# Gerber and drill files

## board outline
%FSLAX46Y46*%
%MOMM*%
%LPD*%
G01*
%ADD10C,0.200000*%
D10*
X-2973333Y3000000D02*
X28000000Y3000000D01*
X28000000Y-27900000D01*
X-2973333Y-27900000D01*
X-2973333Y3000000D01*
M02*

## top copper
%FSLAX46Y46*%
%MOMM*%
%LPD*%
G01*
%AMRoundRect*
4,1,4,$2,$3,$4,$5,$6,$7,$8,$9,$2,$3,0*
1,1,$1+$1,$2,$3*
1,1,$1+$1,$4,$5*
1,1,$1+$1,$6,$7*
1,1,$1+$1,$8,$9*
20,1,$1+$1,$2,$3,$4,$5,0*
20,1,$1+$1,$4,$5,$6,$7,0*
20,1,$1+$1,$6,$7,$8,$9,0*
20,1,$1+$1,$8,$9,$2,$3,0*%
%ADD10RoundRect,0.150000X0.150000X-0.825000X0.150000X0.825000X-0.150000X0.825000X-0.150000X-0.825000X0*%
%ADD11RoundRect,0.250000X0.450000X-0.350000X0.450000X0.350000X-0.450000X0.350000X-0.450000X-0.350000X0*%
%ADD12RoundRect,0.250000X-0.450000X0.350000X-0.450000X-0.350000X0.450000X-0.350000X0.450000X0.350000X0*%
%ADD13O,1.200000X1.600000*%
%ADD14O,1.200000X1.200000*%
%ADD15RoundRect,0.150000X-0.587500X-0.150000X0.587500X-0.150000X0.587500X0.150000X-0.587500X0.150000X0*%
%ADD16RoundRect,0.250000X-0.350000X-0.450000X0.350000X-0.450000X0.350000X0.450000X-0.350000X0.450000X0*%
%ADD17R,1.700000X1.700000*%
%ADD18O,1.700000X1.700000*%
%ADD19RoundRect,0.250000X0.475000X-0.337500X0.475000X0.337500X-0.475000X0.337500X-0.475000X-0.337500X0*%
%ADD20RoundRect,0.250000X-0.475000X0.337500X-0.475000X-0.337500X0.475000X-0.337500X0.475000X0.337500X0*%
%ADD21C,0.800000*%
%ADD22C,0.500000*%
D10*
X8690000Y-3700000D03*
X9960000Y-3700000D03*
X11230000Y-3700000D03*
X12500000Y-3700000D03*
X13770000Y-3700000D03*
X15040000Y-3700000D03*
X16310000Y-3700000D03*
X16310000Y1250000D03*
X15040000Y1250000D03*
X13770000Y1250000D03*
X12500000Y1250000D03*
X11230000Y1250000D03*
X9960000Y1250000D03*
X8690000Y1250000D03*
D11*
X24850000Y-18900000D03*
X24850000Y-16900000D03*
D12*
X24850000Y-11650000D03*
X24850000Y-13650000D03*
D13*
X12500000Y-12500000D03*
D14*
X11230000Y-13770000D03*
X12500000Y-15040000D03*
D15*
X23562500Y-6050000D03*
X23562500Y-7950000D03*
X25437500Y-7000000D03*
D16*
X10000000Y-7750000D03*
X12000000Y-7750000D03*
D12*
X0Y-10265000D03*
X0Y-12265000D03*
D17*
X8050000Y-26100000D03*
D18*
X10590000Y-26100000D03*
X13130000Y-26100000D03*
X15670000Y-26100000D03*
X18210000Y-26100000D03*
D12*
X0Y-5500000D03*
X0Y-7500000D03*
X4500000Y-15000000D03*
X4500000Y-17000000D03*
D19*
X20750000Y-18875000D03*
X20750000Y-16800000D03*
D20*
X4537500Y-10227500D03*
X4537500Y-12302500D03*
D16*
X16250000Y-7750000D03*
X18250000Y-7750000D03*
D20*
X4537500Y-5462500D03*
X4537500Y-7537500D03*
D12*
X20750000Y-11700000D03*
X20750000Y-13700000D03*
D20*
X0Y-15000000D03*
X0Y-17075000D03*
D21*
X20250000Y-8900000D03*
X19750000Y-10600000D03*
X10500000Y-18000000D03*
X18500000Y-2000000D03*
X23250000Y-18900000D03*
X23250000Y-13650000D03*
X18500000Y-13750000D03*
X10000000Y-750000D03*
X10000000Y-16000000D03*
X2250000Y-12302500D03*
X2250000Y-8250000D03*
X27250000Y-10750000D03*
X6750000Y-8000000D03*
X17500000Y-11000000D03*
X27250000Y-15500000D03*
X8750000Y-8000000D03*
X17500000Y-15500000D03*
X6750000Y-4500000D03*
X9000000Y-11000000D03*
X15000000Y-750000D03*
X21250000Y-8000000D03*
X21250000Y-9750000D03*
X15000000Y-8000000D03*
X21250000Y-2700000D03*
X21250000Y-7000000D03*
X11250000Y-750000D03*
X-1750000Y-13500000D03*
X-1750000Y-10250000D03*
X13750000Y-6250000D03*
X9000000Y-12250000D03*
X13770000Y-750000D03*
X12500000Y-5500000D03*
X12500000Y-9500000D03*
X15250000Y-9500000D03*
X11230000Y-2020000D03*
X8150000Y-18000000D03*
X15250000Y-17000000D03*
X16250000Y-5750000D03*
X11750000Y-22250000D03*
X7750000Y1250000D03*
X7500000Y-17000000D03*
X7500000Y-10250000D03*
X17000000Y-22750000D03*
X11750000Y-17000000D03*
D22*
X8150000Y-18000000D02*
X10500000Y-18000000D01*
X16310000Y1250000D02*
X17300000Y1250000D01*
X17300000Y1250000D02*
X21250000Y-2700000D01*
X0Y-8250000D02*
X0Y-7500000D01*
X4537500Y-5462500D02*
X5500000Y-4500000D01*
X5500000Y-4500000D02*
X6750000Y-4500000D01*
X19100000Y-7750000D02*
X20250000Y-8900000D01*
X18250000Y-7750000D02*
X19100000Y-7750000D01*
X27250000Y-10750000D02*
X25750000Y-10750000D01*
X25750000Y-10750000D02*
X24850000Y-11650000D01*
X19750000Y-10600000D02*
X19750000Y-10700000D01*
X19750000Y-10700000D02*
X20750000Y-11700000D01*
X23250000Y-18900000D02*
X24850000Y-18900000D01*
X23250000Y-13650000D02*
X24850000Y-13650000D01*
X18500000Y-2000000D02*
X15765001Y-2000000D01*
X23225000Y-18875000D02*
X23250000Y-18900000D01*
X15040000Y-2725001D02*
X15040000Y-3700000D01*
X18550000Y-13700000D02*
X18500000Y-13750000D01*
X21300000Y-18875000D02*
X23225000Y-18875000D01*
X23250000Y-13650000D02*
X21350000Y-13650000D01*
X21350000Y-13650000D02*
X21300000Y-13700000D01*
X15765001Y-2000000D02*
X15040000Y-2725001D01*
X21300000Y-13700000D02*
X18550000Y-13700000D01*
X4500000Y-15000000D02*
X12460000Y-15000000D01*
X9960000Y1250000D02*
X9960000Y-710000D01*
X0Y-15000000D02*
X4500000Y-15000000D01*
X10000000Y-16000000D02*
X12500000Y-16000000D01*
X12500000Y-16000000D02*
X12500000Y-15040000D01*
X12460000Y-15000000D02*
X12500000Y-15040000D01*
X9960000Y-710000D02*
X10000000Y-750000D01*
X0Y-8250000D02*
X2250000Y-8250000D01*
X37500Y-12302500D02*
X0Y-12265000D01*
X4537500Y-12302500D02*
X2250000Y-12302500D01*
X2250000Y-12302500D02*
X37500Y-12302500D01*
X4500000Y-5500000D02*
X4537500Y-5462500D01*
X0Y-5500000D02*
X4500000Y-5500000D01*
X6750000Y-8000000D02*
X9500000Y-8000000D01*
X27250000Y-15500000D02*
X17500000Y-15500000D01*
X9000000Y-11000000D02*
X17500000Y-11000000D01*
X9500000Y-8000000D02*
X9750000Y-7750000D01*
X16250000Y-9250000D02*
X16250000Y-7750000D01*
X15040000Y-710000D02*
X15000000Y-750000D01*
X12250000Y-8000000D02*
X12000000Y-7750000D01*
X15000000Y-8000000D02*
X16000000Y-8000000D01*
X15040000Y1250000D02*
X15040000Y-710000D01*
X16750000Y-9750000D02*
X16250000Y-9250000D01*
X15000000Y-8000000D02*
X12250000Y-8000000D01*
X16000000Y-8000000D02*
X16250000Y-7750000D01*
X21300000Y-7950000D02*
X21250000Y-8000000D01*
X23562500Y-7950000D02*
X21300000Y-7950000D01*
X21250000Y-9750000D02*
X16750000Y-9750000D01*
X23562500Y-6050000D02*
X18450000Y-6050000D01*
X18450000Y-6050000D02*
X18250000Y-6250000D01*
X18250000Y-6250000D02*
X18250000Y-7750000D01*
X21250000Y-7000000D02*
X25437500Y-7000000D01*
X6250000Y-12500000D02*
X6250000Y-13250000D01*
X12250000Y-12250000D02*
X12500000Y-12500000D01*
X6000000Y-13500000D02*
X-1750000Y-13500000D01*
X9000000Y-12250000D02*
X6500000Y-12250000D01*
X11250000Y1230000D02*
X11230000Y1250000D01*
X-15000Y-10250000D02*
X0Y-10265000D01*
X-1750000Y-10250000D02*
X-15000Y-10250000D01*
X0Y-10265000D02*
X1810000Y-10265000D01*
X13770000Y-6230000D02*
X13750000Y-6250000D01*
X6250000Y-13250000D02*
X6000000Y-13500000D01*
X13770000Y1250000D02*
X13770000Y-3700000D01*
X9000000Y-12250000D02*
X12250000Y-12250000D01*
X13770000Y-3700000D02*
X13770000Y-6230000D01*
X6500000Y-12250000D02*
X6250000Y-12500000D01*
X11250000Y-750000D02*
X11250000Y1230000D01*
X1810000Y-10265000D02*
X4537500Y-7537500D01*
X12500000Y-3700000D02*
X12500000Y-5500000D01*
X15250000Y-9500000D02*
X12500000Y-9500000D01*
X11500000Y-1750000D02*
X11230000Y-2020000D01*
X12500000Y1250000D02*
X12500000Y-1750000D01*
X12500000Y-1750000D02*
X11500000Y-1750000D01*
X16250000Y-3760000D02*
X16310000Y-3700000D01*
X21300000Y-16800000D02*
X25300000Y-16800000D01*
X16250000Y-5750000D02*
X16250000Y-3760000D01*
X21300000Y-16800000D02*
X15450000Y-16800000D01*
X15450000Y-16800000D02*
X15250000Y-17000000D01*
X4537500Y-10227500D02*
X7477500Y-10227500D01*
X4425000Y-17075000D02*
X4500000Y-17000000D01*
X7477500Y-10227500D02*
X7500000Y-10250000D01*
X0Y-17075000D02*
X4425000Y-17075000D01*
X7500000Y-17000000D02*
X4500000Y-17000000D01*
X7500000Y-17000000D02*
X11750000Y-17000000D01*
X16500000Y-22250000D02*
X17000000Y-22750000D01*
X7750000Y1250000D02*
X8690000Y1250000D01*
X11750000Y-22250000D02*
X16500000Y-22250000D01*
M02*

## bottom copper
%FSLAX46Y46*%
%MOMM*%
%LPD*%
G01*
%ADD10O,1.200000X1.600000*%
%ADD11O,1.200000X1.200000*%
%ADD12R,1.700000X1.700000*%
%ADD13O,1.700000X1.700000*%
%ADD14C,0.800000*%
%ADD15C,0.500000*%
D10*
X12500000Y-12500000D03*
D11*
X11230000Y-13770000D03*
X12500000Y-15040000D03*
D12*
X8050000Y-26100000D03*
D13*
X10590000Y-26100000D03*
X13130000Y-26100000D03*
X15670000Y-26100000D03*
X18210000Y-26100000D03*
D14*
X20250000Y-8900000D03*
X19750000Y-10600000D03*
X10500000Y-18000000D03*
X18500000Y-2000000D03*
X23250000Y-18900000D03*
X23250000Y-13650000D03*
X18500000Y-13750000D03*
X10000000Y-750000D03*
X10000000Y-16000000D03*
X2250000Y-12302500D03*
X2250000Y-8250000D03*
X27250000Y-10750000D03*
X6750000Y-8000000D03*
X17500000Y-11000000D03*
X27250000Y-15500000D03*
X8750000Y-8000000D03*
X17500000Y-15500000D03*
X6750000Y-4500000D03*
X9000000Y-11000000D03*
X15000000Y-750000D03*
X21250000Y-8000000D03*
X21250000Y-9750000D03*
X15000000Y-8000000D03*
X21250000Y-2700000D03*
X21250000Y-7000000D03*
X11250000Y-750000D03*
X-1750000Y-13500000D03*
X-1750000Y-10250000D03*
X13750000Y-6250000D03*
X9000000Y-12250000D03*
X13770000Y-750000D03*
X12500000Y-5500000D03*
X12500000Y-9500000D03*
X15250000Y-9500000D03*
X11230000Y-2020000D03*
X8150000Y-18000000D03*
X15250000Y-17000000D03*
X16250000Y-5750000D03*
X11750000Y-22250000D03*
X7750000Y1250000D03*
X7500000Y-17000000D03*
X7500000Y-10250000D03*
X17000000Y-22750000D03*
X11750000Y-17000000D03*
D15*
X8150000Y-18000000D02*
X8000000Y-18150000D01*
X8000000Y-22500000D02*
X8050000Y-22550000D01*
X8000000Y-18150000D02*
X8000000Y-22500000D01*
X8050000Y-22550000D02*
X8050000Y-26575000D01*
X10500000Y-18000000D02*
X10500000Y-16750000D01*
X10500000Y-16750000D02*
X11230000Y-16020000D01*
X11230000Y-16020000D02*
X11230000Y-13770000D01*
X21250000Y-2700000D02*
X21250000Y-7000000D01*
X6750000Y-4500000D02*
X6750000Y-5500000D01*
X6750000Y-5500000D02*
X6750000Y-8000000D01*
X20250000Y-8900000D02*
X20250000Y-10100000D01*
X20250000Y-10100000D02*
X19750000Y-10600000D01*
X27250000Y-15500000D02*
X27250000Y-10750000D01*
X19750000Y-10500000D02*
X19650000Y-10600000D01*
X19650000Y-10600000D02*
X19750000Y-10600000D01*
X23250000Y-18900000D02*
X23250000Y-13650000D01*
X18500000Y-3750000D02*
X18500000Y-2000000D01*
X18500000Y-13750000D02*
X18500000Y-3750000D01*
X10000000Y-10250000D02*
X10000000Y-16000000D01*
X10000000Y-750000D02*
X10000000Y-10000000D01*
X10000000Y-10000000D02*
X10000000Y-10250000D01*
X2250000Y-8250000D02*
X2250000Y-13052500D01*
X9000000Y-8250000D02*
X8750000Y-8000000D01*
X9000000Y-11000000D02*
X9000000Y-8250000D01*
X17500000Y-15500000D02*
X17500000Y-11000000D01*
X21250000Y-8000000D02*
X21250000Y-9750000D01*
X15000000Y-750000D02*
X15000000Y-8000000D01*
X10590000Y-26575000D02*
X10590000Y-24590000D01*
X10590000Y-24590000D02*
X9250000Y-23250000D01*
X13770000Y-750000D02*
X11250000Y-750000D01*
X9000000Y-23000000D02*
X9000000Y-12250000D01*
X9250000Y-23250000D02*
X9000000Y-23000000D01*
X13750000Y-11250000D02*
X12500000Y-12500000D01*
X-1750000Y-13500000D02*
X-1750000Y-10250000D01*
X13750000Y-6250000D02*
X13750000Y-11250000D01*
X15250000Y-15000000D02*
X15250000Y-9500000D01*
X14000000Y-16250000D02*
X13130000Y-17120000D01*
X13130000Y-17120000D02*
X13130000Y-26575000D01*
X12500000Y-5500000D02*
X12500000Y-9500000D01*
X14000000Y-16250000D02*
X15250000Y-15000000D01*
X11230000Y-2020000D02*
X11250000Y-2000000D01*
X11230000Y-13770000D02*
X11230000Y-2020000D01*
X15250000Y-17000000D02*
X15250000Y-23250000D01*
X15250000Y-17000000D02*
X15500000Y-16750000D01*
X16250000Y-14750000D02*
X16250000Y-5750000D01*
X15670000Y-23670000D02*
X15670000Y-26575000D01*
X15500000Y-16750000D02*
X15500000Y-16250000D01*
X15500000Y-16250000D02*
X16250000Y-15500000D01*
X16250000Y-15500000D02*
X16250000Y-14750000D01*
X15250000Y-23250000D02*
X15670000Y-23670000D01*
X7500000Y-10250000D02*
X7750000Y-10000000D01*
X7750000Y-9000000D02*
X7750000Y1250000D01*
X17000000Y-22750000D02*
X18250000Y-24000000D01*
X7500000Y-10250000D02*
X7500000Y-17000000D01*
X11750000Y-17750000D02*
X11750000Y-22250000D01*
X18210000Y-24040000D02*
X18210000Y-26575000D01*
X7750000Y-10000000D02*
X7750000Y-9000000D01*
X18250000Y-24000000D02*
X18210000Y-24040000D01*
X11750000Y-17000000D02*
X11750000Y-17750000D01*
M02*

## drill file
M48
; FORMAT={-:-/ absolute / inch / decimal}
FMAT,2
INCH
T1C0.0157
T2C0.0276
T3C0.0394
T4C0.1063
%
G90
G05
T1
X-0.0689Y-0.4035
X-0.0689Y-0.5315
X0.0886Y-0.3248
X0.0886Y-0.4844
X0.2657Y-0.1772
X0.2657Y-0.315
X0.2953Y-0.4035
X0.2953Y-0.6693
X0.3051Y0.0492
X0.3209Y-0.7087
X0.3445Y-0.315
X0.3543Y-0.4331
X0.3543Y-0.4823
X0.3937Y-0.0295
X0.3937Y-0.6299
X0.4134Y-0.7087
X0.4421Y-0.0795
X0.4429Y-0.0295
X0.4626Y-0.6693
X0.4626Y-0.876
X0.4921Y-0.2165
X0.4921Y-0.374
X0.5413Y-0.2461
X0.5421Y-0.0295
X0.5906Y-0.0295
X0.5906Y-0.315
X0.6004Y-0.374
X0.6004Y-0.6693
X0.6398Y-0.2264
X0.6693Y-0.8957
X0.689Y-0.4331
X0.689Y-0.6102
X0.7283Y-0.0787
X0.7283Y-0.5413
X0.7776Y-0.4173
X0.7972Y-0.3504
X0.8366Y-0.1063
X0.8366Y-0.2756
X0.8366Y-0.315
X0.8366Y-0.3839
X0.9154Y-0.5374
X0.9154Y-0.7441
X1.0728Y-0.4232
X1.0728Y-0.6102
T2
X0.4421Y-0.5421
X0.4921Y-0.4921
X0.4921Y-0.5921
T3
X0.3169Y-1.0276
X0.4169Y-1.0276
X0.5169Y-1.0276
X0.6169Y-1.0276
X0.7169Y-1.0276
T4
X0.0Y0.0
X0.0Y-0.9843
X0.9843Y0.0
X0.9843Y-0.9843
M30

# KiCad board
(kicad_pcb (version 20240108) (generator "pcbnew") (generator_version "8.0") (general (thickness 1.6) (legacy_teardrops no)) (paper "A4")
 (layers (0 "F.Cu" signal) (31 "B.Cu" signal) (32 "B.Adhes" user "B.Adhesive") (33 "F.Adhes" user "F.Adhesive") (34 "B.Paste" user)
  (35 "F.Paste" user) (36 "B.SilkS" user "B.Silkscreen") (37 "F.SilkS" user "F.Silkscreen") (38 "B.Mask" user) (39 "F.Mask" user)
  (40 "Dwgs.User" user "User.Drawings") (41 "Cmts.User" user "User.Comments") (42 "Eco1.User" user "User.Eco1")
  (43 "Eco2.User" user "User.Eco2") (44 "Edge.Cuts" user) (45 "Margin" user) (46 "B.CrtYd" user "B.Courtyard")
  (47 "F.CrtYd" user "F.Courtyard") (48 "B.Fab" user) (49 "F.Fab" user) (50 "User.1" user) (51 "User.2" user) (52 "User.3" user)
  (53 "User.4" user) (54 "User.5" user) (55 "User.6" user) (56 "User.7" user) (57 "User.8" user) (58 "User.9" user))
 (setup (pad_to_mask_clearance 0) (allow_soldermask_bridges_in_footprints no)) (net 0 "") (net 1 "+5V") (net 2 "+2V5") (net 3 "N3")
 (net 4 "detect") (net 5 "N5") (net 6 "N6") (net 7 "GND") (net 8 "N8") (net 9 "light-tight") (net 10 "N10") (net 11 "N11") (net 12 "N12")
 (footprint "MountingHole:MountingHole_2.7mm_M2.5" (layer "F.Cu") (at 0 0)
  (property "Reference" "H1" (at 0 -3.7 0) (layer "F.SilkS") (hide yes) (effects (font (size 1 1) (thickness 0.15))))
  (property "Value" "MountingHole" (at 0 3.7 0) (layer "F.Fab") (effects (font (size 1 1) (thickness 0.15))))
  (pad "" np_thru_hole circle (at 0 0) (size 2.7 2.7) (drill 2.7) (layers "*.Cu" "*.Mask")))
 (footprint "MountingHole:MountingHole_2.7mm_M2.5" (layer "F.Cu") (at 0 25)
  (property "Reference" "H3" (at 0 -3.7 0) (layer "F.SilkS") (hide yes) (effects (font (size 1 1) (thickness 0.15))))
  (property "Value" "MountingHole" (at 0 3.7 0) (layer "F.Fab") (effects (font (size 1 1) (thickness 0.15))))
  (pad "" np_thru_hole circle (at 0 0) (size 2.7 2.7) (drill 2.7) (layers "*.Cu" "*.Mask")))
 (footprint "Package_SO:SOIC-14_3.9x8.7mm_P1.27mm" (layer "F.Cu") (at 12.5 1.225 90)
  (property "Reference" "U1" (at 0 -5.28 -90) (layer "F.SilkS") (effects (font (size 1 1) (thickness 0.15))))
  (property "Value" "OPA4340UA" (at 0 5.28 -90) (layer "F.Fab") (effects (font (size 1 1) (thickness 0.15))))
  (pad "1" smd roundrect (at -2.475 -3.81 90) (size 1.95 0.6) (layers "F.Cu" "F.Paste" "F.Mask") (roundrect_rratio 0.25))
  (pad "2" smd roundrect (at -2.475 -2.54 90) (size 1.95 0.6) (layers "F.Cu" "F.Paste" "F.Mask") (roundrect_rratio 0.25))
  (pad "3" smd roundrect (at -2.475 -1.27 90) (size 1.95 0.6) (layers "F.Cu" "F.Paste" "F.Mask") (roundrect_rratio 0.25))
  (pad "4" smd roundrect (at -2.475 0 90) (size 1.95 0.6) (layers "F.Cu" "F.Paste" "F.Mask") (roundrect_rratio 0.25) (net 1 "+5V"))
  (pad "5" smd roundrect (at -2.475 1.27 90) (size 1.95 0.6) (layers "F.Cu" "F.Paste" "F.Mask") (roundrect_rratio 0.25) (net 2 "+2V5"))
  (pad "6" smd roundrect (at -2.475 2.54 90) (size 1.95 0.6) (layers "F.Cu" "F.Paste" "F.Mask") (roundrect_rratio 0.25) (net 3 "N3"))
  (pad "7" smd roundrect (at -2.475 3.81 90) (size 1.95 0.6) (layers "F.Cu" "F.Paste" "F.Mask") (roundrect_rratio 0.25) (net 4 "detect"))
  (pad "8" smd roundrect (at 2.475 3.81 90) (size 1.95 0.6) (layers "F.Cu" "F.Paste" "F.Mask") (roundrect_rratio 0.25) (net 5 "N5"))
  (pad "9" smd roundrect (at 2.475 2.54 90) (size 1.95 0.6) (layers "F.Cu" "F.Paste" "F.Mask") (roundrect_rratio 0.25) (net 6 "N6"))
  (pad "10" smd roundrect (at 2.475 1.27 90) (size 1.95 0.6) (layers "F.Cu" "F.Paste" "F.Mask") (roundrect_rratio 0.25) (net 2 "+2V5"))
  (pad "11" smd roundrect (at 2.475 0 90) (size 1.95 0.6) (layers "F.Cu" "F.Paste" "F.Mask") (roundrect_rratio 0.25) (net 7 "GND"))
  (pad "12" smd roundrect (at 2.475 -1.27 90) (size 1.95 0.6) (layers "F.Cu" "F.Paste" "F.Mask") (roundrect_rratio 0.25) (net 2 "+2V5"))
  (pad "13" smd roundrect (at 2.475 -2.54 90) (size 1.95 0.6) (layers "F.Cu" "F.Paste" "F.Mask") (roundrect_rratio 0.25) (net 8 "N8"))
  (pad "14" smd roundrect (at 2.475 -3.81 90) (size 1.95 0.6) (layers "F.Cu" "F.Paste" "F.Mask") (roundrect_rratio 0.25)
   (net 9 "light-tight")))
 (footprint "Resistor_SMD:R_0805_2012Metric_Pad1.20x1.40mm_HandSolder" (layer "F.Cu") (at 24.85 17.9 90)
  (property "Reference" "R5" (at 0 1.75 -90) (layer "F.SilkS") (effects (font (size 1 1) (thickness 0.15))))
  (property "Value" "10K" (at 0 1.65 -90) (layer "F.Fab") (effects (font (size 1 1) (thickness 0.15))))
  (pad "1" smd roundrect (at -1 0 90) (size 1.2 1.4) (layers "F.Cu" "F.Paste" "F.Mask") (roundrect_rratio 0.208333) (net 3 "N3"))
  (pad "2" smd roundrect (at 1 0 90) (size 1.2 1.4) (layers "F.Cu" "F.Paste" "F.Mask") (roundrect_rratio 0.208333) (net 4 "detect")))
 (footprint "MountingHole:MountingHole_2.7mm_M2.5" (layer "F.Cu") (at 25 25)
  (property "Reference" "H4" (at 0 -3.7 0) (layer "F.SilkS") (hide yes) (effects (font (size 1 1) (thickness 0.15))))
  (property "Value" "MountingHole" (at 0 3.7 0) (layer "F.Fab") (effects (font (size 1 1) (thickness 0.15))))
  (pad "" np_thru_hole circle (at 0 0) (size 2.7 2.7) (drill 2.7) (layers "*.Cu" "*.Mask")))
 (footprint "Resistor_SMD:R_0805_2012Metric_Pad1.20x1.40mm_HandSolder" (layer "F.Cu") (at 24.85 12.65 -90)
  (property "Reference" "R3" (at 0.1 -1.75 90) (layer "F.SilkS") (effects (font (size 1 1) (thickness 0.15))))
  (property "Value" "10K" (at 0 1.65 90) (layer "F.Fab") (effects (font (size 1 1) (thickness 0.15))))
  (pad "1" smd roundrect (at -1 0 270) (size 1.2 1.4) (layers "F.Cu" "F.Paste" "F.Mask") (roundrect_rratio 0.208333) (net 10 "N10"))
  (pad "2" smd roundrect (at 1 0 270) (size 1.2 1.4) (layers "F.Cu" "F.Paste" "F.Mask") (roundrect_rratio 0.208333) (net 3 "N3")))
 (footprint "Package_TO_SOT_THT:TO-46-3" (layer "F.Cu") (at 12.5 12.5 -90)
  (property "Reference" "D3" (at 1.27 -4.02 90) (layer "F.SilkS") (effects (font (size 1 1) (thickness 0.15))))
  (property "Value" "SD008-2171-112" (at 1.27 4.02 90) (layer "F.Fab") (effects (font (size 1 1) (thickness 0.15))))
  (pad "1" thru_hole oval (at 0 0 270) (size 1.6 1.2) (drill 0.7) (layers "*.Cu" "*.Mask") (remove_unused_layers no) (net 2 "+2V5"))
  (pad "2" thru_hole oval (at 1.27 1.27 270) (size 1.2 1.2) (drill 0.7) (layers "*.Cu" "*.Mask") (remove_unused_layers no) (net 7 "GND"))
  (pad "3" thru_hole oval (at 2.54 0 270) (size 1.2 1.2) (drill 0.7) (layers "*.Cu" "*.Mask") (remove_unused_layers no) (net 8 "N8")))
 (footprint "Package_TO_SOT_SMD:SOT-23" (layer "F.Cu") (at 24.5 7)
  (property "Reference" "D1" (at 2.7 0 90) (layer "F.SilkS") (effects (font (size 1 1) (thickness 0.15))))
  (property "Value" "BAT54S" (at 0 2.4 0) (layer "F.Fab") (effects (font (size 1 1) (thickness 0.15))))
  (pad "1" smd roundrect (at -0.9375 -0.95) (size 1.475 0.6) (layers "F.Cu" "F.Paste" "F.Mask") (roundrect_rratio 0.25) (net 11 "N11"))
  (pad "2" smd roundrect (at -0.9375 0.95) (size 1.475 0.6) (layers "F.Cu" "F.Paste" "F.Mask") (roundrect_rratio 0.25) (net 6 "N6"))
  (pad "3" smd roundrect (at 0.9375 0) (size 1.475 0.6) (layers "F.Cu" "F.Paste" "F.Mask") (roundrect_rratio 0.25) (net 5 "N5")))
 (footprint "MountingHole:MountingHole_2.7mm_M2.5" (layer "F.Cu") (at 25 0)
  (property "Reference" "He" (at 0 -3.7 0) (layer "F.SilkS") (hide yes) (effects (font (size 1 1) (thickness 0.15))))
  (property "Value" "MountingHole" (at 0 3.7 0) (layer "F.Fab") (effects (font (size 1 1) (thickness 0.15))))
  (pad "" np_thru_hole circle (at 0 0) (size 2.7 2.7) (drill 2.7) (layers "*.Cu" "*.Mask")))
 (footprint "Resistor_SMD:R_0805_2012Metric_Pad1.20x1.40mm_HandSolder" (layer "F.Cu") (at 11 7.75)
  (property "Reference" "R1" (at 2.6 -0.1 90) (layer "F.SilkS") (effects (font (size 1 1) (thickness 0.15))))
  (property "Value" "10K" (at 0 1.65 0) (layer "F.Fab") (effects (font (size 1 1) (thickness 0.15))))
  (pad "1" smd roundrect (at -1 0) (size 1.2 1.4) (layers "F.Cu" "F.Paste" "F.Mask") (roundrect_rratio 0.208333) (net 10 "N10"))
  (pad "2" smd roundrect (at 1 0) (size 1.2 1.4) (layers "F.Cu" "F.Paste" "F.Mask") (roundrect_rratio 0.208333) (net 6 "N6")))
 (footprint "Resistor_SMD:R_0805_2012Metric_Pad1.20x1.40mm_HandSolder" (layer "F.Cu") (at 0 11.265 -90)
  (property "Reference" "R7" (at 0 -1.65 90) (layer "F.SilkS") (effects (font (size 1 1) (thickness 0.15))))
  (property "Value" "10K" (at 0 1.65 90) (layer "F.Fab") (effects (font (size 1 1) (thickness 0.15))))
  (pad "1" smd roundrect (at -1 0 270) (size 1.2 1.4) (layers "F.Cu" "F.Paste" "F.Mask") (roundrect_rratio 0.208333) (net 2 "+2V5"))
  (pad "2" smd roundrect (at 1 0 270) (size 1.2 1.4) (layers "F.Cu" "F.Paste" "F.Mask") (roundrect_rratio 0.208333) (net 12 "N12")))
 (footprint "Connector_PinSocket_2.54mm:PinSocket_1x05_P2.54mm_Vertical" (layer "F.Cu") (at 8.05 26.1 90)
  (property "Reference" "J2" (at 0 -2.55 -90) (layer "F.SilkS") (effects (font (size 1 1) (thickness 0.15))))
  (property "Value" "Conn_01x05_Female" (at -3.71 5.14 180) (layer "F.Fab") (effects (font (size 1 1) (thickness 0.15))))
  (pad "1" thru_hole rect (at 0 0 90) (size 1.7 1.7) (drill 1) (layers "*.Cu" "*.Mask") (remove_unused_layers no) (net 7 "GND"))
  (pad "2" thru_hole oval (at 0 2.54 90) (size 1.7 1.7) (drill 1) (layers "*.Cu" "*.Mask") (remove_unused_layers no) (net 2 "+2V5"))
  (pad "3" thru_hole oval (at 0 5.08 90) (size 1.7 1.7) (drill 1) (layers "*.Cu" "*.Mask") (remove_unused_layers no) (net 1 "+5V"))
  (pad "4" thru_hole oval (at 0 7.62 90) (size 1.7 1.7) (drill 1) (layers "*.Cu" "*.Mask") (remove_unused_layers no) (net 4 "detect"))
  (pad "5" thru_hole oval (at 0 10.16 90) (size 1.7 1.7) (drill 1) (layers "*.Cu" "*.Mask") (remove_unused_layers no) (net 9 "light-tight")))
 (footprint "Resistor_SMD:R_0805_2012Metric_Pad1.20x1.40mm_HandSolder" (layer "F.Cu") (at 0 6.5 -90)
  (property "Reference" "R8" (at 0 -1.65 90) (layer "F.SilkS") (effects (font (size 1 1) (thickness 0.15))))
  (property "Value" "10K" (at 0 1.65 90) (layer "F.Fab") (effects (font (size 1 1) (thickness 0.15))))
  (pad "1" smd roundrect (at -1 0 270) (size 1.2 1.4) (layers "F.Cu" "F.Paste" "F.Mask") (roundrect_rratio 0.208333) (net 10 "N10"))
  (pad "2" smd roundrect (at 1 0 270) (size 1.2 1.4) (layers "F.Cu" "F.Paste" "F.Mask") (roundrect_rratio 0.208333) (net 12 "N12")))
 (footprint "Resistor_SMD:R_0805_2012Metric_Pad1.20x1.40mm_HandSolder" (layer "F.Cu") (at 4.5 16 -90)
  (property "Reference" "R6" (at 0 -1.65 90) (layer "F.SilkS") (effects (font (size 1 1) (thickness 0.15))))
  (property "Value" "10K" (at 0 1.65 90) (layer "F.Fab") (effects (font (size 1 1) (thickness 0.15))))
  (pad "1" smd roundrect (at -1 0 270) (size 1.2 1.4) (layers "F.Cu" "F.Paste" "F.Mask") (roundrect_rratio 0.208333) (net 8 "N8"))
  (pad "2" smd roundrect (at 1 0 270) (size 1.2 1.4) (layers "F.Cu" "F.Paste" "F.Mask") (roundrect_rratio 0.208333) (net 9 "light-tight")))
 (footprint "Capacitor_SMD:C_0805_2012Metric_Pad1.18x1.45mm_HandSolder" (layer "F.Cu") (at 20.75 17.8375 90)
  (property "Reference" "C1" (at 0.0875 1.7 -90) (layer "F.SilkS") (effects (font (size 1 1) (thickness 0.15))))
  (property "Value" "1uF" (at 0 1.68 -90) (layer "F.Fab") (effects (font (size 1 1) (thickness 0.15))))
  (pad "1" smd roundrect (at -1.0375 0 90) (size 1.175 1.45) (layers "F.Cu" "F.Paste" "F.Mask") (roundrect_rratio 0.212766) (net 3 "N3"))
  (pad "2" smd roundrect (at 1.0375 0 90) (size 1.175 1.45) (layers "F.Cu" "F.Paste" "F.Mask") (roundrect_rratio 0.212766) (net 4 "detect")))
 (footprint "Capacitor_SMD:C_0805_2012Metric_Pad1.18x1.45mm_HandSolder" (layer "F.Cu") (at 4.5375 11.265 -90)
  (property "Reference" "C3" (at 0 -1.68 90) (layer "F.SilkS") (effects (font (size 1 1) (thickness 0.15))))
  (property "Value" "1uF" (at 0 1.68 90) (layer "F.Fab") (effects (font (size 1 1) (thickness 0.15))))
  (pad "1" smd roundrect (at -1.0375 0 270) (size 1.175 1.45) (layers "F.Cu" "F.Paste" "F.Mask") (roundrect_rratio 0.212766)
   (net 9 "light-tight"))
  (pad "2" smd roundrect (at 1.0375 0 270) (size 1.175 1.45) (layers "F.Cu" "F.Paste" "F.Mask") (roundrect_rratio 0.212766) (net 12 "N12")))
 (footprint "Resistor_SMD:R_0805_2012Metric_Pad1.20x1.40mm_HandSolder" (layer "F.Cu") (at 17.25 7.75)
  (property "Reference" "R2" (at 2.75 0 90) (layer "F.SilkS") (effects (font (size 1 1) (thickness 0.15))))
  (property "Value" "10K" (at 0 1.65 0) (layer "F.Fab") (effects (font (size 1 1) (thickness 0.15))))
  (pad "1" smd roundrect (at -1 0) (size 1.2 1.4) (layers "F.Cu" "F.Paste" "F.Mask") (roundrect_rratio 0.208333) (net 6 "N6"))
  (pad "2" smd roundrect (at 1 0) (size 1.2 1.4) (layers "F.Cu" "F.Paste" "F.Mask") (roundrect_rratio 0.208333) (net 11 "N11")))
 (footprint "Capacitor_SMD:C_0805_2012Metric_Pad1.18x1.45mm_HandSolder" (layer "F.Cu") (at 4.5375 6.5 -90)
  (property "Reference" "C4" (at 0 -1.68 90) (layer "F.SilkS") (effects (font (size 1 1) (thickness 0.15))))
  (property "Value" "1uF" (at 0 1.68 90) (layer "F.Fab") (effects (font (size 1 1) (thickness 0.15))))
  (pad "1" smd roundrect (at -1.0375 0 270) (size 1.175 1.45) (layers "F.Cu" "F.Paste" "F.Mask") (roundrect_rratio 0.212766) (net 10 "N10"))
  (pad "2" smd roundrect (at 1.0375 0 270) (size 1.175 1.45) (layers "F.Cu" "F.Paste" "F.Mask") (roundrect_rratio 0.212766) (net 2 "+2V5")))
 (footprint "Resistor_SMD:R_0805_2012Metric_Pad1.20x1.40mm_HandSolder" (layer "F.Cu") (at 20.75 12.7 -90)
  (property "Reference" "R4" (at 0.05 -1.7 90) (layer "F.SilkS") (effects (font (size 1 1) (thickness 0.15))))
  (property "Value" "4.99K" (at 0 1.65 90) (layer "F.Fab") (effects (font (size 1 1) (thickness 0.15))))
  (pad "1" smd roundrect (at -1 0 270) (size 1.2 1.4) (layers "F.Cu" "F.Paste" "F.Mask") (roundrect_rratio 0.208333) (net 11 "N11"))
  (pad "2" smd roundrect (at 1 0 270) (size 1.2 1.4) (layers "F.Cu" "F.Paste" "F.Mask") (roundrect_rratio 0.208333) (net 3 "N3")))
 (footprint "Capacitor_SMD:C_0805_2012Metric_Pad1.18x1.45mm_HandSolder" (layer "F.Cu") (at 0 16.0375 -90)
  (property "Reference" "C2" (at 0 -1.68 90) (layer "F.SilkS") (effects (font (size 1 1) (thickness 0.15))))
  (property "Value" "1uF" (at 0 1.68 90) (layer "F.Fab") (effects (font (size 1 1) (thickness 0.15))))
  (pad "1" smd roundrect (at -1.0375 0 270) (size 1.175 1.45) (layers "F.Cu" "F.Paste" "F.Mask") (roundrect_rratio 0.212766) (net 8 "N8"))
  (pad "2" smd roundrect (at 1.0375 0 270) (size 1.175 1.45) (layers "F.Cu" "F.Paste" "F.Mask") (roundrect_rratio 0.212766)
   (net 9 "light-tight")))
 (gr_rect (start -2.973333 -3) (end 28 27.9) (stroke (width 0.2) (type default)) (fill none) (layer "Edge.Cuts"))
 (segment (start 23.25 18.9) (end 24.85 18.9) (width 0.5) (layer "F.Cu") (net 3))
 (segment (start 18.5 2) (end 15.765001 2) (width 0.5) (layer "F.Cu") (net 3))
 (segment (start 23.225 18.875) (end 23.25 18.9) (width 0.5) (layer "F.Cu") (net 3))
 (segment (start 15.04 2.725001) (end 15.04 3.7) (width 0.5) (layer "F.Cu") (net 3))
 (segment (start 18.55 13.7) (end 18.5 13.75) (width 0.5) (layer "F.Cu") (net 3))
 (segment (start 23.25 13.65) (end 24.85 13.65) (width 0.5) (layer "F.Cu") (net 3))
 (segment (start 21.3 18.875) (end 23.225 18.875) (width 0.5) (layer "F.Cu") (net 3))
 (segment (start 23.25 13.65) (end 21.35 13.65) (width 0.5) (layer "F.Cu") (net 3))
 (segment (start 21.35 13.65) (end 21.3 13.7) (width 0.5) (layer "F.Cu") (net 3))
 (segment (start 15.765001 2) (end 15.04 2.725001) (width 0.5) (layer "F.Cu") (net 3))
 (segment (start 21.3 13.7) (end 18.55 13.7) (width 0.5) (layer "F.Cu") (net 3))
 (via (at 18.5 2) (size 0.8) (drill 0.4) (layers "F.Cu" "B.Cu") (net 3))
 (via (at 23.25 18.9) (size 0.8) (drill 0.4) (layers "F.Cu" "B.Cu") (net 3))
 (via (at 23.25 13.65) (size 0.8) (drill 0.4) (layers "F.Cu" "B.Cu") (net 3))
 (via (at 18.5 13.75) (size 0.8) (drill 0.4) (layers "F.Cu" "B.Cu") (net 3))
 (segment (start 23.25 18.9) (end 23.25 13.65) (width 0.5) (layer "B.Cu") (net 3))
 (segment (start 18.5 3.75) (end 18.5 2) (width 0.5) (layer "B.Cu") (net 3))
 (segment (start 18.5 13.75) (end 18.5 3.75) (width 0.5) (layer "B.Cu") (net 3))
 (segment (start 4.5 15) (end 12.46 15) (width 0.5) (layer "F.Cu") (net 8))
 (segment (start 9.96 -1.25) (end 9.96 0.71) (width 0.5) (layer "F.Cu") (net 8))
 (segment (start 0 15) (end 4.5 15) (width 0.5) (layer "F.Cu") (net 8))
 (segment (start 10 16) (end 12.5 16) (width 0.5) (layer "F.Cu") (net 8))
 (segment (start 12.5 16) (end 12.5 15.04) (width 0.5) (layer "F.Cu") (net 8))
 (segment (start 12.46 15) (end 12.5 15.04) (width 0.5) (layer "F.Cu") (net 8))
 (segment (start 9.96 0.71) (end 10 0.75) (width 0.5) (layer "F.Cu") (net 8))
 (via (at 10 0.75) (size 0.8) (drill 0.4) (layers "F.Cu" "B.Cu") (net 8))
 (via (at 10 16) (size 0.8) (drill 0.4) (layers "F.Cu" "B.Cu") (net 8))
 (segment (start 10 10.25) (end 10 16) (width 0.5) (layer "B.Cu") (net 8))
 (segment (start 10 0.75) (end 10 10) (width 0.5) (layer "B.Cu") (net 8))
 (segment (start 10 10) (end 10 10.25) (width 0.5) (layer "B.Cu") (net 8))
 (segment (start 0 8.25) (end 2.25 8.25) (width 0.5) (layer "F.Cu") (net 12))
 (segment (start 0 8.25) (end 0 7.5) (width 0.5) (layer "F.Cu") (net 12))
 (segment (start 0.0375 12.3025) (end 0 12.265) (width 0.5) (layer "F.Cu") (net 12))
 (segment (start 4.5375 12.3025) (end 2.25 12.3025) (width 0.5) (layer "F.Cu") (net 12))
 (segment (start 2.25 12.3025) (end 0.0375 12.3025) (width 0.5) (layer "F.Cu") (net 12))
 (via (at 2.25 12.3025) (size 0.8) (drill 0.4) (layers "F.Cu" "B.Cu") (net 12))
 (via (at 2.25 8.25) (size 0.8) (drill 0.4) (layers "F.Cu" "B.Cu") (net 12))
 (segment (start 2.25 8.25) (end 2.25 13.0525) (width 0.5) (layer "B.Cu") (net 12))
 (segment (start 4.5 5.5) (end 4.5375 5.4625) (width 0.5) (layer "F.Cu") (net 10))
 (segment (start 27.25 10.75) (end 25.75 10.75) (width 0.5) (layer "F.Cu") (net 10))
 (segment (start 0 5.5) (end 4.5 5.5) (width 0.5) (layer "F.Cu") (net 10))
 (segment (start 6.75 8) (end 9.5 8) (width 0.5) (layer "F.Cu") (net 10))
 (segment (start 25.75 10.75) (end 24.85 11.65) (width 0.5) (layer "F.Cu") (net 10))
 (segment (start 27.25 15.5) (end 17.5 15.5) (width 0.5) (layer "F.Cu") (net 10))
 (segment (start 4.5375 5.4625) (end 5.5 4.5) (width 0.5) (layer "F.Cu") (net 10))
 (segment (start 9 11) (end 17.5 11) (width 0.5) (layer "F.Cu") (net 10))
 (segment (start 9.5 8) (end 9.75 7.75) (width 0.5) (layer "F.Cu") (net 10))
 (segment (start 5.5 4.5) (end 6.75 4.5) (width 0.5) (layer "F.Cu") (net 10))
 (via (at 27.25 10.75) (size 0.8) (drill 0.4) (layers "F.Cu" "B.Cu") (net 10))
 (via (at 6.75 8) (size 0.8) (drill 0.4) (layers "F.Cu" "B.Cu") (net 10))
 (via (at 17.5 11) (size 0.8) (drill 0.4) (layers "F.Cu" "B.Cu") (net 10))
 (via (at 27.25 15.5) (size 0.8) (drill 0.4) (layers "F.Cu" "B.Cu") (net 10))
 (via (at 8.75 8) (size 0.8) (drill 0.4) (layers "F.Cu" "B.Cu") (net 10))
 (via (at 17.5 15.5) (size 0.8) (drill 0.4) (layers "F.Cu" "B.Cu") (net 10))
 (via (at 6.75 4.5) (size 0.8) (drill 0.4) (layers "F.Cu" "B.Cu") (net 10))
 (via (at 9 11) (size 0.8) (drill 0.4) (layers "F.Cu" "B.Cu") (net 10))
 (segment (start 6.75 5.5) (end 6.75 8) (width 0.5) (layer "B.Cu") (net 10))
 (segment (start 6.75 4.5) (end 6.75 5.5) (width 0.5) (layer "B.Cu") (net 10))
 (segment (start 9 8.25) (end 8.75 8) (width 0.5) (layer "B.Cu") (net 10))
 (segment (start 27.25 15.5) (end 27.25 10.75) (width 0.5) (layer "B.Cu") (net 10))
 (segment (start 9 11) (end 9 8.25) (width 0.5) (layer "B.Cu") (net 10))
 (segment (start 17.5 15.5) (end 17.5 11) (width 0.5) (layer "B.Cu") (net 10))
 (segment (start 16.25 9.25) (end 16.25 7.75) (width 0.5) (layer "F.Cu") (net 6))
 (segment (start 15.04 0.71) (end 15 0.75) (width 0.5) (layer "F.Cu") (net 6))
 (segment (start 12.25 8) (end 12 7.75) (width 0.5) (layer "F.Cu") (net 6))
 (segment (start 15 8) (end 16 8) (width 0.5) (layer "F.Cu") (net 6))
 (segment (start 15.04 -1.25) (end 15.04 0.71) (width 0.5) (layer "F.Cu") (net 6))
 (segment (start 16.75 9.75) (end 16.25 9.25) (width 0.5) (layer "F.Cu") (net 6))
 (segment (start 15 8) (end 12.25 8) (width 0.5) (layer "F.Cu") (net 6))
 (segment (start 16 8) (end 16.25 7.75) (width 0.5) (layer "F.Cu") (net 6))
 (segment (start 21.3 7.95) (end 21.25 8) (width 0.5) (layer "F.Cu") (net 6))
 (segment (start 23.5625 7.95) (end 21.3 7.95) (width 0.5) (layer "F.Cu") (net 6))
 (segment (start 21.25 9.75) (end 16.75 9.75) (width 0.5) (layer "F.Cu") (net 6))
 (via (at 15 0.75) (size 0.8) (drill 0.4) (layers "F.Cu" "B.Cu") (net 6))
 (via (at 21.25 8) (size 0.8) (drill 0.4) (layers "F.Cu" "B.Cu") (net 6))
 (via (at 21.25 9.75) (size 0.8) (drill 0.4) (layers "F.Cu" "B.Cu") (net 6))
 (via (at 15 8) (size 0.8) (drill 0.4) (layers "F.Cu" "B.Cu") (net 6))
 (segment (start 21.25 8) (end 21.25 9.75) (width 0.5) (layer "B.Cu") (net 6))
 (segment (start 15 0.75) (end 15 8) (width 0.5) (layer "B.Cu") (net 6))
 (segment (start 23.5625 6.05) (end 18.45 6.05) (width 0.5) (layer "F.Cu") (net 11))
 (segment (start 19.75 10.7) (end 20.75 11.7) (width 0.5) (layer "F.Cu") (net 11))
 (segment (start 18.25 7.75) (end 19.1 7.75) (width 0.5) (layer "F.Cu") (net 11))
 (segment (start 18.45 6.05) (end 18.25 6.25) (width 0.5) (layer "F.Cu") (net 11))
 (segment (start 18.25 6.25) (end 18.25 7.75) (width 0.5) (layer "F.Cu") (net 11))
 (segment (start 19.75 10.6) (end 19.75 10.7) (width 0.5) (layer "F.Cu") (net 11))
 (segment (start 19.1 7.75) (end 20.25 8.9) (width 0.5) (layer "F.Cu") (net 11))
 (via (at 19.75 10.6) (size 0.8) (drill 0.4) (layers "F.Cu" "B.Cu") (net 11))
 (via (at 20.25 8.9) (size 0.8) (drill 0.4) (layers "F.Cu" "B.Cu") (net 11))
 (segment (start 20.25 10.1) (end 19.75 10.6) (width 0.5) (layer "B.Cu") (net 11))
 (segment (start 19.75 10.5) (end 19.65 10.6) (width 0.5) (layer "B.Cu") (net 11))
 (segment (start 20.25 8.9) (end 20.25 10.1) (width 0.5) (layer "B.Cu") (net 11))
 (segment (start 19.65 10.6) (end 19.75 10.6) (width 0.5) (layer "B.Cu") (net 11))
 (segment (start 21.25 7) (end 25.4375 7) (width 0.5) (layer "F.Cu") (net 5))
 (segment (start 16.31 -1.25) (end 17.3 -1.25) (width 0.5) (layer "F.Cu") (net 5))
 (segment (start 17.3 -1.25) (end 21.25 2.7) (width 0.5) (layer "F.Cu") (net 5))
 (via (at 21.25 2.7) (size 0.8) (drill 0.4) (layers "F.Cu" "B.Cu") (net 5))
 (via (at 21.25 7) (size 0.8) (drill 0.4) (layers "F.Cu" "B.Cu") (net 5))
 (segment (start 21.25 2.7) (end 21.25 7) (width 0.5) (layer "B.Cu") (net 5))
 (segment (start 6.25 12.5) (end 6.25 13.25) (width 0.5) (layer "F.Cu") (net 2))
 (segment (start 12.25 12.25) (end 12.5 12.5) (width 0.5) (layer "F.Cu") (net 2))
 (segment (start 6 13.5) (end -1.75 13.5) (width 0.5) (layer "F.Cu") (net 2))
 (segment (start 9 12.25) (end 6.5 12.25) (width 0.5) (layer "F.Cu") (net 2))
 (segment (start 11.25 -1.23) (end 11.23 -1.25) (width 0.5) (layer "F.Cu") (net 2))
 (segment (start -0.015 10.25) (end 0 10.265) (width 0.5) (layer "F.Cu") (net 2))
 (segment (start -1.75 10.25) (end -0.015 10.25) (width 0.5) (layer "F.Cu") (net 2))
 (segment (start 0 10.265) (end 1.81 10.265) (width 0.5) (layer "F.Cu") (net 2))
 (segment (start 13.77 6.23) (end 13.75 6.25) (width 0.5) (layer "F.Cu") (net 2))
 (segment (start 6.25 13.25) (end 6 13.5) (width 0.5) (layer "F.Cu") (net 2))
 (segment (start 13.77 -1.25) (end 13.77 3.7) (width 0.5) (layer "F.Cu") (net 2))
 (segment (start 9 12.25) (end 12.25 12.25) (width 0.5) (layer "F.Cu") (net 2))
 (segment (start 13.77 3.7) (end 13.77 6.23) (width 0.5) (layer "F.Cu") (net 2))
 (segment (start 6.5 12.25) (end 6.25 12.5) (width 0.5) (layer "F.Cu") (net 2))
 (segment (start 11.25 0.75) (end 11.25 -1.23) (width 0.5) (layer "F.Cu") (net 2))
 (segment (start 1.81 10.265) (end 4.5375 7.5375) (width 0.5) (layer "F.Cu") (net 2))
 (via (at 11.25 0.75) (size 0.8) (drill 0.4) (layers "F.Cu" "B.Cu") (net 2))
 (via (at -1.75 13.5) (size 0.8) (drill 0.4) (layers "F.Cu" "B.Cu") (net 2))
 (via (at -1.75 10.25) (size 0.8) (drill 0.4) (layers "F.Cu" "B.Cu") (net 2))
 (via (at 13.75 6.25) (size 0.8) (drill 0.4) (layers "F.Cu" "B.Cu") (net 2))
 (via (at 9 12.25) (size 0.8) (drill 0.4) (layers "F.Cu" "B.Cu") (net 2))
 (via (at 13.77 0.75) (size 0.8) (drill 0.4) (layers "F.Cu" "B.Cu") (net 2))
 (segment (start 10.59 26.575) (end 10.59 24.59) (width 0.5) (layer "B.Cu") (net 2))
 (segment (start 10.59 24.59) (end 9.25 23.25) (width 0.5) (layer "B.Cu") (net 2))
 (segment (start 13.77 0.75) (end 11.25 0.75) (width 0.5) (layer "B.Cu") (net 2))
 (segment (start 9 23) (end 9 12.25) (width 0.5) (layer "B.Cu") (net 2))
 (segment (start 9.25 23.25) (end 9 23) (width 0.5) (layer "B.Cu") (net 2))
 (segment (start 13.75 11.25) (end 12.5 12.5) (width 0.5) (layer "B.Cu") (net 2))
 (segment (start -1.75 13.5) (end -1.75 10.25) (width 0.5) (layer "B.Cu") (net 2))
 (segment (start 13.75 6.25) (end 13.75 11.25) (width 0.5) (layer "B.Cu") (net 2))
 (segment (start 12.5 3.7) (end 12.5 5.5) (width 0.5) (layer "F.Cu") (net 1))
 (segment (start 15.25 9.5) (end 12.5 9.5) (width 0.5) (layer "F.Cu") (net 1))
 (via (at 12.5 5.5) (size 0.8) (drill 0.4) (layers "F.Cu" "B.Cu") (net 1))
 (via (at 12.5 9.5) (size 0.8) (drill 0.4) (layers "F.Cu" "B.Cu") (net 1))
 (via (at 15.25 9.5) (size 0.8) (drill 0.4) (layers "F.Cu" "B.Cu") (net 1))
 (segment (start 15.25 15) (end 15.25 9.5) (width 0.5) (layer "B.Cu") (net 1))
 (segment (start 14 16.25) (end 13.13 17.12) (width 0.5) (layer "B.Cu") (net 1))
 (segment (start 13.13 17.12) (end 13.13 26.575) (width 0.5) (layer "B.Cu") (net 1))
 (segment (start 12.5 5.5) (end 12.5 9.5) (width 0.5) (layer "B.Cu") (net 1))
 (segment (start 14 16.25) (end 15.25 15) (width 0.5) (layer "B.Cu") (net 1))
 (segment (start 11.5 1.75) (end 11.23 2.02) (width 0.5) (layer "F.Cu") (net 7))
 (segment (start 8.15 18) (end 10.5 18) (width 0.5) (layer "F.Cu") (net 7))
 (segment (start 12.5 -1.25) (end 12.5 1.75) (width 0.5) (layer "F.Cu") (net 7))
 (segment (start 12.5 1.75) (end 11.5 1.75) (width 0.5) (layer "F.Cu") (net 7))
 (via (at 11.23 2.02) (size 0.8) (drill 0.4) (layers "F.Cu" "B.Cu") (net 7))
 (via (at 10.5 18) (size 0.8) (drill 0.4) (layers "F.Cu" "B.Cu") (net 7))
 (via (at 8.15 18) (size 0.8) (drill 0.4) (layers "F.Cu" "B.Cu") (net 7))
 (segment (start 8 22.5) (end 8.05 22.55) (width 0.5) (layer "B.Cu") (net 7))
 (segment (start 11.23 2.02) (end 11.25 2) (width 0.5) (layer "B.Cu") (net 7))
 (segment (start 11.23 13.77) (end 11.23 2.02) (width 0.5) (layer "B.Cu") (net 7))
 (segment (start 8.05 22.55) (end 8.05 26.575) (width 0.5) (layer "B.Cu") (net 7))
 (segment (start 11.23 16.02) (end 11.23 13.77) (width 0.5) (layer "B.Cu") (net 7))
 (segment (start 10.5 18) (end 10.5 16.75) (width 0.5) (layer "B.Cu") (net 7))
 (segment (start 8.15 18) (end 8 18.15) (width 0.5) (layer "B.Cu") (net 7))
 (segment (start 10.5 16.75) (end 11.23 16.02) (width 0.5) (layer "B.Cu") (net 7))
 (segment (start 8 18.15) (end 8 22.5) (width 0.5) (layer "B.Cu") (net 7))
 (segment (start 16.25 3.76) (end 16.31 3.7) (width 0.5) (layer "F.Cu") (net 4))
 (segment (start 21.3 16.8) (end 25.3 16.8) (width 0.5) (layer "F.Cu") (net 4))
 (segment (start 16.25 5.75) (end 16.25 3.76) (width 0.5) (layer "F.Cu") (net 4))
 (segment (start 21.3 16.8) (end 15.45 16.8) (width 0.5) (layer "F.Cu") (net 4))
 (segment (start 15.45 16.8) (end 15.25 17) (width 0.5) (layer "F.Cu") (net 4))
 (via (at 15.25 17) (size 0.8) (drill 0.4) (layers "F.Cu" "B.Cu") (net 4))
 (via (at 16.25 5.75) (size 0.8) (drill 0.4) (layers "F.Cu" "B.Cu") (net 4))
 (segment (start 15.25 17) (end 15.25 23.25) (width 0.5) (layer "B.Cu") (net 4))
 (segment (start 15.25 17) (end 15.5 16.75) (width 0.5) (layer "B.Cu") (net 4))
 (segment (start 16.25 14.75) (end 16.25 5.75) (width 0.5) (layer "B.Cu") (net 4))
 (segment (start 15.67 23.67) (end 15.67 26.575) (width 0.5) (layer "B.Cu") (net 4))
 (segment (start 15.5 16.75) (end 15.5 16.25) (width 0.5) (layer "B.Cu") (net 4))
 (segment (start 15.5 16.25) (end 16.25 15.5) (width 0.5) (layer "B.Cu") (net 4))
 (segment (start 16.25 15.5) (end 16.25 14.75) (width 0.5) (layer "B.Cu") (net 4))
 (segment (start 15.25 23.25) (end 15.67 23.67) (width 0.5) (layer "B.Cu") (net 4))
 (segment (start 4.5375 10.2275) (end 7.4775 10.2275) (width 0.5) (layer "F.Cu") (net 9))
 (segment (start 4.425 17.075) (end 4.5 17) (width 0.5) (layer "F.Cu") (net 9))
 (segment (start 7.4775 10.2275) (end 7.5 10.25) (width 0.5) (layer "F.Cu") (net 9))
 (segment (start 0 17.075) (end 4.425 17.075) (width 0.5) (layer "F.Cu") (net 9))
 (segment (start 7.5 17) (end 4.5 17) (width 0.5) (layer "F.Cu") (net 9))
 (segment (start 7.5 17) (end 11.75 17) (width 0.5) (layer "F.Cu") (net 9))
 (segment (start 16.5 22.25) (end 17 22.75) (width 0.5) (layer "F.Cu") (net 9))
 (segment (start 7.75 -1.25) (end 8.69 -1.25) (width 0.5) (layer "F.Cu") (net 9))
 (segment (start 11.75 22.25) (end 16.5 22.25) (width 0.5) (layer "F.Cu") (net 9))
 (via (at 11.75 22.25) (size 0.8) (drill 0.4) (layers "F.Cu" "B.Cu") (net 9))
 (via (at 7.75 -1.25) (size 0.8) (drill 0.4) (layers "F.Cu" "B.Cu") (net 9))
 (via (at 7.5 17) (size 0.8) (drill 0.4) (layers "F.Cu" "B.Cu") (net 9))
 (via (at 7.5 10.25) (size 0.8) (drill 0.4) (layers "F.Cu" "B.Cu") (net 9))
 (via (at 17 22.75) (size 0.8) (drill 0.4) (layers "F.Cu" "B.Cu") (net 9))
 (via (at 11.75 17) (size 0.8) (drill 0.4) (layers "F.Cu" "B.Cu") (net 9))
 (segment (start 7.5 10.25) (end 7.75 10) (width 0.5) (layer "B.Cu") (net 9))
 (segment (start 7.75 9) (end 7.75 -1.25) (width 0.5) (layer "B.Cu") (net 9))
 (segment (start 17 22.75) (end 18.25 24) (width 0.5) (layer "B.Cu") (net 9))
 (segment (start 7.5 10.25) (end 7.5 17) (width 0.5) (layer "B.Cu") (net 9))
 (segment (start 11.75 17.75) (end 11.75 22.25) (width 0.5) (layer "B.Cu") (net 9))
 (segment (start 18.21 24.04) (end 18.21 26.575) (width 0.5) (layer "B.Cu") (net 9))
 (segment (start 7.75 10) (end 7.75 9) (width 0.5) (layer "B.Cu") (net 9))
 (segment (start 18.25 24) (end 18.21 24.04) (width 0.5) (layer "B.Cu") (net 9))
 (segment (start 11.75 17) (end 11.75 17.75) (width 0.5) (layer "B.Cu") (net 9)))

